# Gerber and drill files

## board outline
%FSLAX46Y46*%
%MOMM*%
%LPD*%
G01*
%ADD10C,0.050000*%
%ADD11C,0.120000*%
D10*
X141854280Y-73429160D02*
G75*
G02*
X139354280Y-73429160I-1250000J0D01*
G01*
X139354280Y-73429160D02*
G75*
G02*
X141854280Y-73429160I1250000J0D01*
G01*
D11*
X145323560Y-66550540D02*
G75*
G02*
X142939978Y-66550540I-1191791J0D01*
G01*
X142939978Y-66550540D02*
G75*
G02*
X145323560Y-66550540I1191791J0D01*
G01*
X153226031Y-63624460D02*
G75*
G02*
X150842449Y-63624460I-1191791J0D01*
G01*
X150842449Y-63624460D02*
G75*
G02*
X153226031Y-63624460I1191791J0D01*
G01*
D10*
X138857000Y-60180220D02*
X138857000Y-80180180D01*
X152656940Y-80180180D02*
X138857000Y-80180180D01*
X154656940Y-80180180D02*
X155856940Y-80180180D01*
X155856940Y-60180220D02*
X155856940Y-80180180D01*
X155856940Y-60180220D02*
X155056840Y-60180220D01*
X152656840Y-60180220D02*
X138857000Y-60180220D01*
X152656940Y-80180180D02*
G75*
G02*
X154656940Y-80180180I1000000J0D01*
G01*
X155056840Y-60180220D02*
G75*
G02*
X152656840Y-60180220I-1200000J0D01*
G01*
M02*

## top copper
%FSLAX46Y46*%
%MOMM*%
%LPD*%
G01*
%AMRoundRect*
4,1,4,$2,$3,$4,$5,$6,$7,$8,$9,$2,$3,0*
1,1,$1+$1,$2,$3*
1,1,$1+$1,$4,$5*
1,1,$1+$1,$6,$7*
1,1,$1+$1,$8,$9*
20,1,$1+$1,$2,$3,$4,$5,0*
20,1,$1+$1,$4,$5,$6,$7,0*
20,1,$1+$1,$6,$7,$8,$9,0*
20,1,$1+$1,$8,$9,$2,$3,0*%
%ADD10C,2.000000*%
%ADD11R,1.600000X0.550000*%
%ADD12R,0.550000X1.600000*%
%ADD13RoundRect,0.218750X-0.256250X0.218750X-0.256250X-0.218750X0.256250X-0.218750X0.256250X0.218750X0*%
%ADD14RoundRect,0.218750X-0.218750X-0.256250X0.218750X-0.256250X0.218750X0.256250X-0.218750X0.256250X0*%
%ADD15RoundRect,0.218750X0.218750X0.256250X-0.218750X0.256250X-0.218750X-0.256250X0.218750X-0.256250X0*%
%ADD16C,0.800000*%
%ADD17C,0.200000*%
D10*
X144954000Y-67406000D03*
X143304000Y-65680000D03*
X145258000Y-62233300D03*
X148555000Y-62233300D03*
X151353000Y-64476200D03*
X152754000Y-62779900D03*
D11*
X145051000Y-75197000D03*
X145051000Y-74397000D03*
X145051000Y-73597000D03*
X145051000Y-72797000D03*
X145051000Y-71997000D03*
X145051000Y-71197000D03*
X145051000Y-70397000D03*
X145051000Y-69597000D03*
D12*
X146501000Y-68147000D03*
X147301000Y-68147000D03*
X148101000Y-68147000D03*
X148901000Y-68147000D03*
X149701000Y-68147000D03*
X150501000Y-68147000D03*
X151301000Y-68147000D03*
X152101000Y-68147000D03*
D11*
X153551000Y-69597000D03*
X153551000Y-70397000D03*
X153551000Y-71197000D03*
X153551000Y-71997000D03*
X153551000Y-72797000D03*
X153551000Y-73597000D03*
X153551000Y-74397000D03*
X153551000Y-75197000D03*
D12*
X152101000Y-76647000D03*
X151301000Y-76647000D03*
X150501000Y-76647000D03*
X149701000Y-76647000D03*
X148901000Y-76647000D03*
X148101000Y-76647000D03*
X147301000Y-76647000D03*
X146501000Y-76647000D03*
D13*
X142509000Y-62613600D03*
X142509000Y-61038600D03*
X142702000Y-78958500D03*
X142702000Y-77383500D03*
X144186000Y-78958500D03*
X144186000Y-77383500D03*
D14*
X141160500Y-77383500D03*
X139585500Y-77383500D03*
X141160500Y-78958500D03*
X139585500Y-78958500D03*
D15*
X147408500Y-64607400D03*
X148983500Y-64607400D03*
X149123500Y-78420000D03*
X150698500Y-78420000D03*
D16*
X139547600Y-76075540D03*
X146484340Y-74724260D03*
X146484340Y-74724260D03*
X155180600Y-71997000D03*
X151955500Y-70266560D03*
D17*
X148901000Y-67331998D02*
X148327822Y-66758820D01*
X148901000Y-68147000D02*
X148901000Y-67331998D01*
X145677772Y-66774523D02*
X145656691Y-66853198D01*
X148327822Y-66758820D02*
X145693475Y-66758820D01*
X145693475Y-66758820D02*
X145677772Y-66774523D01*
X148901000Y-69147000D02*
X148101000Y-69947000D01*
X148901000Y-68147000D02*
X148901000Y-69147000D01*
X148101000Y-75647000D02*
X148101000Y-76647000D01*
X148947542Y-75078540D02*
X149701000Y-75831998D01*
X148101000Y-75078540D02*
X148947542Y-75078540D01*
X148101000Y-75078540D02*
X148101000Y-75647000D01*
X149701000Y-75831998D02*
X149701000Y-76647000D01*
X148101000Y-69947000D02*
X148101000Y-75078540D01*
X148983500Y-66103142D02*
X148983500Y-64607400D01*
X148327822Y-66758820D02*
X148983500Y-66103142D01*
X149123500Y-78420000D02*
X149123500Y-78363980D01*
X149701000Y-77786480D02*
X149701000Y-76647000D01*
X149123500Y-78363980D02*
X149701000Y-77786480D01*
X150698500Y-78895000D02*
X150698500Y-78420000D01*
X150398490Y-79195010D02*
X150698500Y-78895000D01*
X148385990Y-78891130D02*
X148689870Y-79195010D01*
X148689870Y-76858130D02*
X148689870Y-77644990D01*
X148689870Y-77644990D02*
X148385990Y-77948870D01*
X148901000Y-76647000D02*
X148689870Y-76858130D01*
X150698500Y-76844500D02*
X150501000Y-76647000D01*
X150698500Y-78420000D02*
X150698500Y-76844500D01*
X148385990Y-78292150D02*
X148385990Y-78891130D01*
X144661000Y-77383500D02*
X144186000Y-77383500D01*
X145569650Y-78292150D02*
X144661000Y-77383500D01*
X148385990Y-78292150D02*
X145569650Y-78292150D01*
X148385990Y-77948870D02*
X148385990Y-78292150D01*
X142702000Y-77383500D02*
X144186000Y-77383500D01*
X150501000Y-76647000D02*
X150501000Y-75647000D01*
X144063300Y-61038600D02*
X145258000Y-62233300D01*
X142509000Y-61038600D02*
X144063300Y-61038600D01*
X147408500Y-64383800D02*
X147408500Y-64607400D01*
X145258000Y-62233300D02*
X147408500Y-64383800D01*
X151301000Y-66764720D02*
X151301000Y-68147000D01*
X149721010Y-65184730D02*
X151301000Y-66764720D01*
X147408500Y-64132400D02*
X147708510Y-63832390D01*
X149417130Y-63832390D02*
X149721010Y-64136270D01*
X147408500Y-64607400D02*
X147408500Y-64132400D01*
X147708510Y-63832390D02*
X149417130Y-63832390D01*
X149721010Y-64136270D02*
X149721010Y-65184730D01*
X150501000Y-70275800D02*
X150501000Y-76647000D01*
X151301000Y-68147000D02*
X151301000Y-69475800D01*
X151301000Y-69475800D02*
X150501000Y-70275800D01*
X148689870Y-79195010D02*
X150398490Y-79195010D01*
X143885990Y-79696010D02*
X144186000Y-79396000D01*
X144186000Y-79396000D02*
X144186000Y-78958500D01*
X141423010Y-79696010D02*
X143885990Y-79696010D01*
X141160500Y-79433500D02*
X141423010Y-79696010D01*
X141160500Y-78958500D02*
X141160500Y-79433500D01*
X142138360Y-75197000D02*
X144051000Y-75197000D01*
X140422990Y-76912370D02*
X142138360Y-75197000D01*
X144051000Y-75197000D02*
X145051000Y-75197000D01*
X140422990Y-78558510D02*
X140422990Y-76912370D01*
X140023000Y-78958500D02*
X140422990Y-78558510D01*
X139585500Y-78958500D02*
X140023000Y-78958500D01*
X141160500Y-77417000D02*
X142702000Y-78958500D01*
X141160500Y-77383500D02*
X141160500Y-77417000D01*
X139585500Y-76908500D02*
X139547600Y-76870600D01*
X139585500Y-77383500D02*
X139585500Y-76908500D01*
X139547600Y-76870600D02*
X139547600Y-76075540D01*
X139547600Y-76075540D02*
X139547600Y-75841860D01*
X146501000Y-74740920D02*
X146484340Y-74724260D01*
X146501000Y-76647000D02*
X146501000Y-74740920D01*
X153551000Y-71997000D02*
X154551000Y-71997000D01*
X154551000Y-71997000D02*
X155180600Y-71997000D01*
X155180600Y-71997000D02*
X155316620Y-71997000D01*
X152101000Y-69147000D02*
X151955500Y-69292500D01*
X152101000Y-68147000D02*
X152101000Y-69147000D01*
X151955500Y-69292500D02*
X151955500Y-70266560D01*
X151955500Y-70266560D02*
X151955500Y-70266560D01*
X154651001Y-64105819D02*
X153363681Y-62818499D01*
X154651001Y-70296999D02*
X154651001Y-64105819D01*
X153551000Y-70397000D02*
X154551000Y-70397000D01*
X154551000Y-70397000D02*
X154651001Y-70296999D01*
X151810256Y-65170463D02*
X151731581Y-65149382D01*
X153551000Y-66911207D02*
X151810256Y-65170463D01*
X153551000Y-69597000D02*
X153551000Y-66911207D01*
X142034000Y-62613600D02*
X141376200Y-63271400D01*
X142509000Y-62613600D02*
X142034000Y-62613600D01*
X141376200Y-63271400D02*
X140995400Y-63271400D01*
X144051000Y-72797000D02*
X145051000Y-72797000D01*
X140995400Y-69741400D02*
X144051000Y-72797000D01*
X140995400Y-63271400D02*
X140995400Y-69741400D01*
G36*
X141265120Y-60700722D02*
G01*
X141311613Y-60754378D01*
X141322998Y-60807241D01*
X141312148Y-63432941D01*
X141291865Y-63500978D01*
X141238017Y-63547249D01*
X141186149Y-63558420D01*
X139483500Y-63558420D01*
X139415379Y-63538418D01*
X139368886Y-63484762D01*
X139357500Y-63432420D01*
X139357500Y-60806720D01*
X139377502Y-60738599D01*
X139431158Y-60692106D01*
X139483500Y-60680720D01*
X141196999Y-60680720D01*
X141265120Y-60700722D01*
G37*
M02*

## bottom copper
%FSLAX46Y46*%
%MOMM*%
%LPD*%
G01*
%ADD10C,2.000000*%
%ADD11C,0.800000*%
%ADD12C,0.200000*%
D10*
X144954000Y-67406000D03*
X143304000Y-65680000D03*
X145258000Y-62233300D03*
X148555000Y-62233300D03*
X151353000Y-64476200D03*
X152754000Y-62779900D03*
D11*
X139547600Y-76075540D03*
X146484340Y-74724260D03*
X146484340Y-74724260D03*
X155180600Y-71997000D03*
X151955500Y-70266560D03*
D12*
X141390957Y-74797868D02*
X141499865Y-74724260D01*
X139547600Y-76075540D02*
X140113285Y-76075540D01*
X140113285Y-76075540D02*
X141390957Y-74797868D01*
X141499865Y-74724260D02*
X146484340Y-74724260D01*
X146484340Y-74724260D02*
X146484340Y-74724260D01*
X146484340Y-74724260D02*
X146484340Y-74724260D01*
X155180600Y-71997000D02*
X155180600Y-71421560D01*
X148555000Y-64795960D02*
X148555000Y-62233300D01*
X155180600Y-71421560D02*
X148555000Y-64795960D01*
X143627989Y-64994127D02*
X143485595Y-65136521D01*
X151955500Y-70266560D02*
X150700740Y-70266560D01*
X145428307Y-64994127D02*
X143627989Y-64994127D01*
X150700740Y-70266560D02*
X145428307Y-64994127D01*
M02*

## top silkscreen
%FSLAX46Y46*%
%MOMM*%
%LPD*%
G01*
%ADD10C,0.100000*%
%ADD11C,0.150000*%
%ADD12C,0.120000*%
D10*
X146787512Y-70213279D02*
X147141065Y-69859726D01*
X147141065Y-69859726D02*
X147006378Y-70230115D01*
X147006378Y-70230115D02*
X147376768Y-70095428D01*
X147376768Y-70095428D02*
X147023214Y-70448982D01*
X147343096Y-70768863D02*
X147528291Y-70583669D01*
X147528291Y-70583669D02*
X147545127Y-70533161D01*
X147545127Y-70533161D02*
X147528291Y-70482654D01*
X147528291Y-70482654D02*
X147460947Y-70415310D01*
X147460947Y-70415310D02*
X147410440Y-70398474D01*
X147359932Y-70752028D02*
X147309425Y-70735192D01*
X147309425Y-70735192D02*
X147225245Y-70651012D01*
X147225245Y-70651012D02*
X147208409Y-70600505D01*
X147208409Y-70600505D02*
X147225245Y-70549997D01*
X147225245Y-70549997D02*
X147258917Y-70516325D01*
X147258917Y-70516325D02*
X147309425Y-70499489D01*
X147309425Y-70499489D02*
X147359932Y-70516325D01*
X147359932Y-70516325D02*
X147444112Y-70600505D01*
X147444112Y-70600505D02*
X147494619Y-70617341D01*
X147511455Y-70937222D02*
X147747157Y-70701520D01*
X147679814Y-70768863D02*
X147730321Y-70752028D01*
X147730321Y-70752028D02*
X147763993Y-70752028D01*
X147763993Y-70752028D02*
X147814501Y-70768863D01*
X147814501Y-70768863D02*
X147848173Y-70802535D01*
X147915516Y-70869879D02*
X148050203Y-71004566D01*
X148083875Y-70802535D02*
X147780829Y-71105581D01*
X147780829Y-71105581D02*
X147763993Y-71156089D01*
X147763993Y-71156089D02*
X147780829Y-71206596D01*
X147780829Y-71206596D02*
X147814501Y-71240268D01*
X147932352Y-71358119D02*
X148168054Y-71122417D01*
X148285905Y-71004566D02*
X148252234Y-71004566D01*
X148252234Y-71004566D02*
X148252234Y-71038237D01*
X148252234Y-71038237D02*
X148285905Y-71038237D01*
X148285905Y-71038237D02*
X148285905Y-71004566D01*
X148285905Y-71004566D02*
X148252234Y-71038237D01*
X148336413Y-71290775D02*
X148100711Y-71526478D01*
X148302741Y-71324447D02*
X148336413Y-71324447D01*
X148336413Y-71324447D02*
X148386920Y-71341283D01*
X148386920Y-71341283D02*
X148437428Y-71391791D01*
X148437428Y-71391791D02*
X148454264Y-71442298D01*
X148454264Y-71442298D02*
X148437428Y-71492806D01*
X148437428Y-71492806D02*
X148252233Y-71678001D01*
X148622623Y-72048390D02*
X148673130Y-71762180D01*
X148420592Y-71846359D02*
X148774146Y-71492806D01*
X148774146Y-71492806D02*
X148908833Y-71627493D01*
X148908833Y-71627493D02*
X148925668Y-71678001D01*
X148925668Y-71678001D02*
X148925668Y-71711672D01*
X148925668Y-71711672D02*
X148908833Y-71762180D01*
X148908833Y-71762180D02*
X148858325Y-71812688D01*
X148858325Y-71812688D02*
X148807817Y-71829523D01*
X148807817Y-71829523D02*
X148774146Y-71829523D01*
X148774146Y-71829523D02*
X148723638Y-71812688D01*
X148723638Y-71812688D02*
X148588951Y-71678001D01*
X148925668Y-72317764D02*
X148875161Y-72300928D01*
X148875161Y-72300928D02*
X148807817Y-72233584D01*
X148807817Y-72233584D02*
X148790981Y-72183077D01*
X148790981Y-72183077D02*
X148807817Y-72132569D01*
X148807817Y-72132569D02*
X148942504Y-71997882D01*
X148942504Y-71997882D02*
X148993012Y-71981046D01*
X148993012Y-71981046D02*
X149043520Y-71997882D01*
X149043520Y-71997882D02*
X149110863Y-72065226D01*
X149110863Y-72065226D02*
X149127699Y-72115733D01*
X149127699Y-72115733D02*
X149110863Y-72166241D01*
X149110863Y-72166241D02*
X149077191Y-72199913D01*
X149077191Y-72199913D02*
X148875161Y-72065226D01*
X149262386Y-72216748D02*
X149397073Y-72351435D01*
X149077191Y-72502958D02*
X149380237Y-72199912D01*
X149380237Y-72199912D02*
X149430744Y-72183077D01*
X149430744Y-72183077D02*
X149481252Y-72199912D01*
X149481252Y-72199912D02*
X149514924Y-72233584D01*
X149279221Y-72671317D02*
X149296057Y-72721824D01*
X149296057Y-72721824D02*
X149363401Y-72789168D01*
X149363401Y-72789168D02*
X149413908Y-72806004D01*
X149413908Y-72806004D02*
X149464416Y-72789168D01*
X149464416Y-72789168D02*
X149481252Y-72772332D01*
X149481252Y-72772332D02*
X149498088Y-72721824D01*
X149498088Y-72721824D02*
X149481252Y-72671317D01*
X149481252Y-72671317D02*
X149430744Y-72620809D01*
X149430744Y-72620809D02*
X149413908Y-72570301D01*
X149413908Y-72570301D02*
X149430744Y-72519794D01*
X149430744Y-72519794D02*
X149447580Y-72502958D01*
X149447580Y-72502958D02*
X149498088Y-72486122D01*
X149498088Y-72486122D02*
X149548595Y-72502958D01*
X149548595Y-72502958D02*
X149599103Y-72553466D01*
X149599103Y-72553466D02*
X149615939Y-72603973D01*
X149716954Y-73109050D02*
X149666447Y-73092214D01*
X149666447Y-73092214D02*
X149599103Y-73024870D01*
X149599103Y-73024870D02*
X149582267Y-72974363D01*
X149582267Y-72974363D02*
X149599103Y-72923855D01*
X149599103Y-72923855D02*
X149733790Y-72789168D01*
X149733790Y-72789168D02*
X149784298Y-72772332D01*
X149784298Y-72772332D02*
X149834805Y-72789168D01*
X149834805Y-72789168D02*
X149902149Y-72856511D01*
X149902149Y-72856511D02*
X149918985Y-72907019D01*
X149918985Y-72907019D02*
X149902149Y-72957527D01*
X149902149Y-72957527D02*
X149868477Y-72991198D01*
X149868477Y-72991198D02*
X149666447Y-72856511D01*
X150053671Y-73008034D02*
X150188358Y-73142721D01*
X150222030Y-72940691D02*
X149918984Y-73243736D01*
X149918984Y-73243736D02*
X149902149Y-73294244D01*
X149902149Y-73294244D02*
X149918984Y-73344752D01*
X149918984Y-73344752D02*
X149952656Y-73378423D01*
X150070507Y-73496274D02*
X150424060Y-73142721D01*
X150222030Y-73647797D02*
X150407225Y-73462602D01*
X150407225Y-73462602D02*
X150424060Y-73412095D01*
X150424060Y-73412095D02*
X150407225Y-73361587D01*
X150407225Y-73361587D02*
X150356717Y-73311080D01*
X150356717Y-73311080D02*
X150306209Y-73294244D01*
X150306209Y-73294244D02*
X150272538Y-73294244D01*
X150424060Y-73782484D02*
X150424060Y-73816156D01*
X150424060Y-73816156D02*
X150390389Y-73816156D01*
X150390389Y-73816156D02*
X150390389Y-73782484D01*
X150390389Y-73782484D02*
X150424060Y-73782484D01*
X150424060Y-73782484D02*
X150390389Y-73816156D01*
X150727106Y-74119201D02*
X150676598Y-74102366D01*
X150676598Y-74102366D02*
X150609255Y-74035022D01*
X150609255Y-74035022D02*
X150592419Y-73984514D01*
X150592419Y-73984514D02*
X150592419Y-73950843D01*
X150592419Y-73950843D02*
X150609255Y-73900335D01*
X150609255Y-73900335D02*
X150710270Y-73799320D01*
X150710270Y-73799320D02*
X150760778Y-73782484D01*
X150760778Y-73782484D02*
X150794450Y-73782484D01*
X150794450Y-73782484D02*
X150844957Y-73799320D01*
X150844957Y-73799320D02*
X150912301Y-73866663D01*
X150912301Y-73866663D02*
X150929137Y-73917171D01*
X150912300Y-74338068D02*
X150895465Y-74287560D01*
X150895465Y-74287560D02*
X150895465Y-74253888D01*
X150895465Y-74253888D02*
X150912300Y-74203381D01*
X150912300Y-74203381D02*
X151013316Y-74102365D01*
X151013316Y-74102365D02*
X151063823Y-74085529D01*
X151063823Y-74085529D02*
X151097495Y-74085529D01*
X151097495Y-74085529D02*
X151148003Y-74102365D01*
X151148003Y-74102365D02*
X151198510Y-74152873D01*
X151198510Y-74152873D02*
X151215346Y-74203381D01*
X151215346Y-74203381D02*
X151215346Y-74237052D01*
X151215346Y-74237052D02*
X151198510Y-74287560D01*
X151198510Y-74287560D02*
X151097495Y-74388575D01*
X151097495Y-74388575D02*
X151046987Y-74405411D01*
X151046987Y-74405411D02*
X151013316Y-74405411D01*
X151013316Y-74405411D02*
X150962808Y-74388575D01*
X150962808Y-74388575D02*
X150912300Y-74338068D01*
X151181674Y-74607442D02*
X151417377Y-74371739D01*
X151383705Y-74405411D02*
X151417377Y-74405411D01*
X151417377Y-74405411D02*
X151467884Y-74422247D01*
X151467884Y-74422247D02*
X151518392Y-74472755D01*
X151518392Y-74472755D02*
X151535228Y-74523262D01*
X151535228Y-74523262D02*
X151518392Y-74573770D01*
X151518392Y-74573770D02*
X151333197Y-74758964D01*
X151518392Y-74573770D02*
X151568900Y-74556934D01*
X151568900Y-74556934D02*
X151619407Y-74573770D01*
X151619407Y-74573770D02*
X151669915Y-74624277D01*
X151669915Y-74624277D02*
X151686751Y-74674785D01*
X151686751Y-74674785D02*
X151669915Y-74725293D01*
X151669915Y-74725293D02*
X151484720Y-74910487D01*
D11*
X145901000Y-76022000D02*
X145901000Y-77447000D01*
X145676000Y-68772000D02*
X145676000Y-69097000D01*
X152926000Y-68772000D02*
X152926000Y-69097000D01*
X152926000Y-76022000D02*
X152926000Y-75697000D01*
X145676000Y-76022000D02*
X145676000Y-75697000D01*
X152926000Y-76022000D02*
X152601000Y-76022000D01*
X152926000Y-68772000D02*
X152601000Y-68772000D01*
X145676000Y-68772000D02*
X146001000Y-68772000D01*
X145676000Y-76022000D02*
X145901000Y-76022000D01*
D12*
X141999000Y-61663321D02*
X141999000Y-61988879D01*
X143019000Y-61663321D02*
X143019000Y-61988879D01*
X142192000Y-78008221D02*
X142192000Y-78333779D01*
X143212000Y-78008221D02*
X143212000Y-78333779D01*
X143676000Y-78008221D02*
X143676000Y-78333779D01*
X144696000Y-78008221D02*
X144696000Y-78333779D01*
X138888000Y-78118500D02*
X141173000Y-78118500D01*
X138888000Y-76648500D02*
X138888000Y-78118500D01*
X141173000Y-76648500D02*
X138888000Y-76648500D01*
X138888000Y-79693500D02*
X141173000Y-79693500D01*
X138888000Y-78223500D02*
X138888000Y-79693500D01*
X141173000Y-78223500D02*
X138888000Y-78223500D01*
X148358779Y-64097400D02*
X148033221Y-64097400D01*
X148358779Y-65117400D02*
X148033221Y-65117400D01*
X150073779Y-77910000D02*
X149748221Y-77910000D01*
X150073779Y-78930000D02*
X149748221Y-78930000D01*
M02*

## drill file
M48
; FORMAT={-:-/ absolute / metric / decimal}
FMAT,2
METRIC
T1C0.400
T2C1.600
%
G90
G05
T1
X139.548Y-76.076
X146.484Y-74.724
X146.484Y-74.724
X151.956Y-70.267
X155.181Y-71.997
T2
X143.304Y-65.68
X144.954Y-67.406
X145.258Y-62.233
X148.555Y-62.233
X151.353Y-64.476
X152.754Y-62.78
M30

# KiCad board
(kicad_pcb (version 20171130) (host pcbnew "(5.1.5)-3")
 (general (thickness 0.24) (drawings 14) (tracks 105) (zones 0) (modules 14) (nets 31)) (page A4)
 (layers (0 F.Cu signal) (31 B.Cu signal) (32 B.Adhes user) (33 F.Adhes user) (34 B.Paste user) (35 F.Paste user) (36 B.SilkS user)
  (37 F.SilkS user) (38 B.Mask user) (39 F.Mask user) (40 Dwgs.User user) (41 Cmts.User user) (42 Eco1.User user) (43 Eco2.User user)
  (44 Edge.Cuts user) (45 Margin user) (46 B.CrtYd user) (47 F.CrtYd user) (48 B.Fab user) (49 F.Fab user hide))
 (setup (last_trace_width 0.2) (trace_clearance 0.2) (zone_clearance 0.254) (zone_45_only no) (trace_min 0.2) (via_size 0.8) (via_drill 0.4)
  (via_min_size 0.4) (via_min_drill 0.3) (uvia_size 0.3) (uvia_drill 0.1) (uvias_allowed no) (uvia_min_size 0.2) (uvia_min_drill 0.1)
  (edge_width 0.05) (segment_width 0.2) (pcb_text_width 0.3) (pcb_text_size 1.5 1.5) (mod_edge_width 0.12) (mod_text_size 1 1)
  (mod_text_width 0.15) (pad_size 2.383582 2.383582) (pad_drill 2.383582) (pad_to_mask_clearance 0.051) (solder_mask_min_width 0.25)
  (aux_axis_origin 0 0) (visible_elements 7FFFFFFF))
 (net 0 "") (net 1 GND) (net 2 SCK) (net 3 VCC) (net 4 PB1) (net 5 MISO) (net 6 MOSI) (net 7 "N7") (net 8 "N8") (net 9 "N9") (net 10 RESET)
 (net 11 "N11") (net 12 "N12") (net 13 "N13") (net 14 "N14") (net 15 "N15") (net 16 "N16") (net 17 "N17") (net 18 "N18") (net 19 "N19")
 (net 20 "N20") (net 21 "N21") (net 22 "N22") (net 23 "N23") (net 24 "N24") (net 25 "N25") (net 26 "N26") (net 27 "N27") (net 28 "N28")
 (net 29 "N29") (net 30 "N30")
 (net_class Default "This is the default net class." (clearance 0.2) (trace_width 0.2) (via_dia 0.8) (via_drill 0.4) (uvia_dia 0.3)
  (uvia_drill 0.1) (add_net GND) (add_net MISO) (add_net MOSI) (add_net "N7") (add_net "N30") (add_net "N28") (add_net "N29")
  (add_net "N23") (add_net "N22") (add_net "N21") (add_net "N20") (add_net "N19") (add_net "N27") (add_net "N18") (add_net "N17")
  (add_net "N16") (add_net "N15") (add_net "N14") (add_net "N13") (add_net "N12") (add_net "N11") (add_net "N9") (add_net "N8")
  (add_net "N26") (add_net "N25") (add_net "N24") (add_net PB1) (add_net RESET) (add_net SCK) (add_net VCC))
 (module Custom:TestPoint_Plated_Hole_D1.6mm (layer F.Cu) (at 144.954 67.406 180)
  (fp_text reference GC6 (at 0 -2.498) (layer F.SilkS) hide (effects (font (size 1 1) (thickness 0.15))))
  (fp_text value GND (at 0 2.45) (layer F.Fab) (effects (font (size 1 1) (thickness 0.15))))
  (pad 1 thru_hole circle (at 0 0 180) (size 2 2) (drill 1.6) (layers *.Cu *.Mask) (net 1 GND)))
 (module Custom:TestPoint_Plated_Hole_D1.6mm (layer F.Cu) (at 143.304 65.68 180)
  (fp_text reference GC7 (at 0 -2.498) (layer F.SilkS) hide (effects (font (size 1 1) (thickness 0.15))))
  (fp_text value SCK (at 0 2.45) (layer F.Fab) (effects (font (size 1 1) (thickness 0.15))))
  (pad 1 thru_hole circle (at 0 0 180) (size 2 2) (drill 1.6) (layers *.Cu *.Mask) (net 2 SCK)))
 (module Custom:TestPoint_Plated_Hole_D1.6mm (layer F.Cu) (at 145.258 62.2333 180)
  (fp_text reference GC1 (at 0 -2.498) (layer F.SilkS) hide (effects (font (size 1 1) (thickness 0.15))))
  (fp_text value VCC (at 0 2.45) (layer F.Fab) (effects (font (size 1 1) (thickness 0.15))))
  (pad 1 thru_hole circle (at 0 0 180) (size 2 2) (drill 1.6) (layers *.Cu *.Mask) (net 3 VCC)))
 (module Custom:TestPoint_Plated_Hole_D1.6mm (layer F.Cu) (at 148.555 62.2333 180)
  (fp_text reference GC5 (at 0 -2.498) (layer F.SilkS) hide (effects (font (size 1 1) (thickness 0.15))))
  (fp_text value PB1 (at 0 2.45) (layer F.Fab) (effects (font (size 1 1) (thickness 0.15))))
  (pad 1 thru_hole circle (at 0 0 180) (size 2 2) (drill 1.6) (layers *.Cu *.Mask) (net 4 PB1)))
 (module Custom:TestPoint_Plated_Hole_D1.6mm (layer F.Cu) (at 151.353 64.4762 180)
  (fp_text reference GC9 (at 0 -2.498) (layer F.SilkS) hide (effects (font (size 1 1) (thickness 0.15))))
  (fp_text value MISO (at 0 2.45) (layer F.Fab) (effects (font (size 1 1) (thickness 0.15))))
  (pad 1 thru_hole circle (at 0 0 180) (size 2 2) (drill 1.6) (layers *.Cu *.Mask) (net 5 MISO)))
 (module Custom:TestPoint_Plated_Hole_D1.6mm (layer F.Cu) (at 152.754 62.7799 180)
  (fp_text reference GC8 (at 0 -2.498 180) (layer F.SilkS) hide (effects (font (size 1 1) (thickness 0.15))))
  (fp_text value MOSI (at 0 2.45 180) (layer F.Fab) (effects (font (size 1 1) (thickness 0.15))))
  (pad 1 thru_hole circle (at 0 0 180) (size 2 2) (drill 1.6) (layers *.Cu *.Mask) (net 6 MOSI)))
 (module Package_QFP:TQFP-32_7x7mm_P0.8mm (layer F.Cu) (at 149.301 72.397 90)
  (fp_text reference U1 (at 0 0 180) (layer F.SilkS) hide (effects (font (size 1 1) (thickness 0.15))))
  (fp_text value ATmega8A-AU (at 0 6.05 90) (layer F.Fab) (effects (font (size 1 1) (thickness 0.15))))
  (fp_line (start -3.625 -3.4) (end -5.05 -3.4) (layer F.SilkS) (width 0.15))
  (fp_line (start 3.625 -3.625) (end 3.3 -3.625) (layer F.SilkS) (width 0.15))
  (fp_line (start 3.625 3.625) (end 3.3 3.625) (layer F.SilkS) (width 0.15))
  (fp_line (start -3.625 3.625) (end -3.3 3.625) (layer F.SilkS) (width 0.15))
  (fp_line (start -3.625 -3.625) (end -3.3 -3.625) (layer F.SilkS) (width 0.15))
  (fp_line (start -3.625 3.625) (end -3.625 3.3) (layer F.SilkS) (width 0.15))
  (fp_line (start 3.625 3.625) (end 3.625 3.3) (layer F.SilkS) (width 0.15))
  (fp_line (start 3.625 -3.625) (end 3.625 -3.3) (layer F.SilkS) (width 0.15))
  (fp_line (start -3.625 -3.625) (end -3.625 -3.4) (layer F.SilkS) (width 0.15))
  (pad 32 smd rect (at -2.8 -4.25 180) (size 1.6 0.55) (layers F.Cu F.Paste F.Mask) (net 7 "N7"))
  (pad 31 smd rect (at -2 -4.25 180) (size 1.6 0.55) (layers F.Cu F.Paste F.Mask) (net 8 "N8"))
  (pad 30 smd rect (at -1.2 -4.25 180) (size 1.6 0.55) (layers F.Cu F.Paste F.Mask) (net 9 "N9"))
  (pad 29 smd rect (at -0.4 -4.25 180) (size 1.6 0.55) (layers F.Cu F.Paste F.Mask) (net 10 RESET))
  (pad 28 smd rect (at 0.4 -4.25 180) (size 1.6 0.55) (layers F.Cu F.Paste F.Mask) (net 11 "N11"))
  (pad 27 smd rect (at 1.2 -4.25 180) (size 1.6 0.55) (layers F.Cu F.Paste F.Mask) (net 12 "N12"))
  (pad 26 smd rect (at 2 -4.25 180) (size 1.6 0.55) (layers F.Cu F.Paste F.Mask) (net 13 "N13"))
  (pad 25 smd rect (at 2.8 -4.25 180) (size 1.6 0.55) (layers F.Cu F.Paste F.Mask) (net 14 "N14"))
  (pad 24 smd rect (at 4.25 -2.8 90) (size 1.6 0.55) (layers F.Cu F.Paste F.Mask) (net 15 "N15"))
  (pad 23 smd rect (at 4.25 -2 90) (size 1.6 0.55) (layers F.Cu F.Paste F.Mask) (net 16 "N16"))
  (pad 22 smd rect (at 4.25 -1.2 90) (size 1.6 0.55) (layers F.Cu F.Paste F.Mask) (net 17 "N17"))
  (pad 21 smd rect (at 4.25 -0.4 90) (size 1.6 0.55) (layers F.Cu F.Paste F.Mask) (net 1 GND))
  (pad 20 smd rect (at 4.25 0.4 90) (size 1.6 0.55) (layers F.Cu F.Paste F.Mask) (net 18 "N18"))
  (pad 19 smd rect (at 4.25 1.2 90) (size 1.6 0.55) (layers F.Cu F.Paste F.Mask) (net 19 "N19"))
  (pad 18 smd rect (at 4.25 2 90) (size 1.6 0.55) (layers F.Cu F.Paste F.Mask) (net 3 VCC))
  (pad 17 smd rect (at 4.25 2.8 90) (size 1.6 0.55) (layers F.Cu F.Paste F.Mask) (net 2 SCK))
  (pad 16 smd rect (at 2.8 4.25 180) (size 1.6 0.55) (layers F.Cu F.Paste F.Mask) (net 5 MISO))
  (pad 15 smd rect (at 2 4.25 180) (size 1.6 0.55) (layers F.Cu F.Paste F.Mask) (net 6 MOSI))
  (pad 14 smd rect (at 1.2 4.25 180) (size 1.6 0.55) (layers F.Cu F.Paste F.Mask) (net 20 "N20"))
  (pad 13 smd rect (at 0.4 4.25 180) (size 1.6 0.55) (layers F.Cu F.Paste F.Mask) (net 4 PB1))
  (pad 12 smd rect (at -0.4 4.25 180) (size 1.6 0.55) (layers F.Cu F.Paste F.Mask) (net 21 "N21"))
  (pad 11 smd rect (at -1.2 4.25 180) (size 1.6 0.55) (layers F.Cu F.Paste F.Mask) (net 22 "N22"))
  (pad 10 smd rect (at -2 4.25 180) (size 1.6 0.55) (layers F.Cu F.Paste F.Mask) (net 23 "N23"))
  (pad 9 smd rect (at -2.8 4.25 180) (size 1.6 0.55) (layers F.Cu F.Paste F.Mask) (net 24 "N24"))
  (pad 8 smd rect (at -4.25 2.8 90) (size 1.6 0.55) (layers F.Cu F.Paste F.Mask) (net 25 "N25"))
  (pad 7 smd rect (at -4.25 2 90) (size 1.6 0.55) (layers F.Cu F.Paste F.Mask) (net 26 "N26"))
  (pad 6 smd rect (at -4.25 1.2 90) (size 1.6 0.55) (layers F.Cu F.Paste F.Mask) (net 3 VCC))
  (pad 5 smd rect (at -4.25 0.4 90) (size 1.6 0.55) (layers F.Cu F.Paste F.Mask) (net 1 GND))
  (pad 4 smd rect (at -4.25 -0.4 90) (size 1.6 0.55) (layers F.Cu F.Paste F.Mask) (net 3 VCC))
  (pad 3 smd rect (at -4.25 -1.2 90) (size 1.6 0.55) (layers F.Cu F.Paste F.Mask) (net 1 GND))
  (pad 2 smd rect (at -4.25 -2 90) (size 1.6 0.55) (layers F.Cu F.Paste F.Mask) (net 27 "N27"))
  (pad 1 smd rect (at -4.25 -2.8 90) (size 1.6 0.55) (layers F.Cu F.Paste F.Mask) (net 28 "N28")))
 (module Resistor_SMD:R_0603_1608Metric (layer F.Cu) (at 142.509 61.8261 270)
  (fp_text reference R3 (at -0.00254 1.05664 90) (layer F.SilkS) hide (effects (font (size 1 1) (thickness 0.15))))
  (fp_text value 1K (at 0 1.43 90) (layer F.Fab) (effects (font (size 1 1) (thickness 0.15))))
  (fp_line (start -0.162779 0.51) (end 0.162779 0.51) (layer F.SilkS) (width 0.12))
  (fp_line (start -0.162779 -0.51) (end 0.162779 -0.51) (layer F.SilkS) (width 0.12))
  (pad 2 smd roundrect (at 0.7875 0 270) (size 0.875 0.95) (layers F.Cu F.Paste F.Mask) (roundrect_rratio 0.25) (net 10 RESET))
  (pad 1 smd roundrect (at -0.7875 0 270) (size 0.875 0.95) (layers F.Cu F.Paste F.Mask) (roundrect_rratio 0.25) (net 3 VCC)))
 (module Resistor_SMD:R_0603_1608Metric (layer F.Cu) (at 142.702 78.171 270)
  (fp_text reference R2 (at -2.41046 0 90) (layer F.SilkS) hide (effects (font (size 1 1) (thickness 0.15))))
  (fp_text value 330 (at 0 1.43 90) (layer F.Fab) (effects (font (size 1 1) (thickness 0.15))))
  (fp_line (start -0.162779 0.51) (end 0.162779 0.51) (layer F.SilkS) (width 0.12))
  (fp_line (start -0.162779 -0.51) (end 0.162779 -0.51) (layer F.SilkS) (width 0.12))
  (pad 2 smd roundrect (at 0.7875 0 270) (size 0.875 0.95) (layers F.Cu F.Paste F.Mask) (roundrect_rratio 0.25) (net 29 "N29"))
  (pad 1 smd roundrect (at -0.7875 0 270) (size 0.875 0.95) (layers F.Cu F.Paste F.Mask) (roundrect_rratio 0.25) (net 3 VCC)))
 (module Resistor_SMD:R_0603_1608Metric (layer F.Cu) (at 144.186 78.171 270)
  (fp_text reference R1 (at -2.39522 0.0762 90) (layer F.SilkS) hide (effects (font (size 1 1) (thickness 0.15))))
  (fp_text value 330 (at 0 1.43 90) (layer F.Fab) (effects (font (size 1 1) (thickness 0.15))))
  (fp_line (start -0.162779 0.51) (end 0.162779 0.51) (layer F.SilkS) (width 0.12))
  (fp_line (start -0.162779 -0.51) (end 0.162779 -0.51) (layer F.SilkS) (width 0.12))
  (pad 2 smd roundrect (at 0.7875 0 270) (size 0.875 0.95) (layers F.Cu F.Paste F.Mask) (roundrect_rratio 0.25) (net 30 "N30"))
  (pad 1 smd roundrect (at -0.7875 0 270) (size 0.875 0.95) (layers F.Cu F.Paste F.Mask) (roundrect_rratio 0.25) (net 3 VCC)))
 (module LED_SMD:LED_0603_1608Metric (layer F.Cu) (at 140.373 77.3835)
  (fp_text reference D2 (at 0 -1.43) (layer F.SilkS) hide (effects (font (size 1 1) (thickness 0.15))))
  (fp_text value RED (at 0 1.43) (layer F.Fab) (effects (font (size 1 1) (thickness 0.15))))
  (fp_line (start -1.485 0.735) (end 0.8 0.735) (layer F.SilkS) (width 0.12))
  (fp_line (start -1.485 -0.735) (end -1.485 0.735) (layer F.SilkS) (width 0.12))
  (fp_line (start 0.8 -0.735) (end -1.485 -0.735) (layer F.SilkS) (width 0.12))
  (pad 2 smd roundrect (at 0.7875 0) (size 0.875 0.95) (layers F.Cu F.Paste F.Mask) (roundrect_rratio 0.25) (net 29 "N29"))
  (pad 1 smd roundrect (at -0.7875 0) (size 0.875 0.95) (layers F.Cu F.Paste F.Mask) (roundrect_rratio 0.25) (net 28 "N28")))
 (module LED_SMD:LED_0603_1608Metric (layer F.Cu) (at 140.373 78.9585)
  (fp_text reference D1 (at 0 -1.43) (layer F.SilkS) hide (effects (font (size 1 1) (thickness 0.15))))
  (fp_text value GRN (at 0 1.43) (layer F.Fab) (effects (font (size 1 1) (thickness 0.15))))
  (fp_line (start -1.485 0.735) (end 0.8 0.735) (layer F.SilkS) (width 0.12))
  (fp_line (start -1.485 -0.735) (end -1.485 0.735) (layer F.SilkS) (width 0.12))
  (fp_line (start 0.8 -0.735) (end -1.485 -0.735) (layer F.SilkS) (width 0.12))
  (pad 2 smd roundrect (at 0.7875 0) (size 0.875 0.95) (layers F.Cu F.Paste F.Mask) (roundrect_rratio 0.25) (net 30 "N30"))
  (pad 1 smd roundrect (at -0.7875 0) (size 0.875 0.95) (layers F.Cu F.Paste F.Mask) (roundrect_rratio 0.25) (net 7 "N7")))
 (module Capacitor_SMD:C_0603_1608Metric (layer F.Cu) (at 148.196 64.6074 180)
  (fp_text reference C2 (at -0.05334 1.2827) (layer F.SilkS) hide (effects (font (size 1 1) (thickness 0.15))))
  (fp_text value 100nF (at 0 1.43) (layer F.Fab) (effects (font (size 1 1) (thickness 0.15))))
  (fp_line (start -0.162779 0.51) (end 0.162779 0.51) (layer F.SilkS) (width 0.12))
  (fp_line (start -0.162779 -0.51) (end 0.162779 -0.51) (layer F.SilkS) (width 0.12))
  (pad 2 smd roundrect (at 0.7875 0 180) (size 0.875 0.95) (layers F.Cu F.Paste F.Mask) (roundrect_rratio 0.25) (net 3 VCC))
  (pad 1 smd roundrect (at -0.7875 0 180) (size 0.875 0.95) (layers F.Cu F.Paste F.Mask) (roundrect_rratio 0.25) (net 1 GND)))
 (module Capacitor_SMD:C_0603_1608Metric (layer F.Cu) (at 149.911 78.42 180)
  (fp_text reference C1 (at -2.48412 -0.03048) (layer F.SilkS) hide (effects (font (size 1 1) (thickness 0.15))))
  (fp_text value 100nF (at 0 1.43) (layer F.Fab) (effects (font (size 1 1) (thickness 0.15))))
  (fp_line (start -0.162779 0.51) (end 0.162779 0.51) (layer F.SilkS) (width 0.12))
  (fp_line (start -0.162779 -0.51) (end 0.162779 -0.51) (layer F.SilkS) (width 0.12))
  (pad 2 smd roundrect (at 0.7875 0 180) (size 0.875 0.95) (layers F.Cu F.Paste F.Mask) (roundrect_rratio 0.25) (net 1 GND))
  (pad 1 smd roundrect (at -0.7875 0 180) (size 0.875 0.95) (layers F.Cu F.Paste F.Mask) (roundrect_rratio 0.25) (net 3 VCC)))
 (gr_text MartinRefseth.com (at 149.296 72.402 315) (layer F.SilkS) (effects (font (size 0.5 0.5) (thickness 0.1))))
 (gr_circle (center 140.60428 73.42916) (end 140.60428 74.67916) (layer Edge.Cuts) (width 0.05))
 (gr_circle (center 144.131769 66.55054) (end 144.131769 65.358749) (layer Edge.Cuts) (width 0.12))
 (gr_circle (center 152.03424 63.62446) (end 152.03424 62.432669) (layer Edge.Cuts) (width 0.12))
 (gr_line (start 138.857 60.18022) (end 138.857 80.18018) (layer Edge.Cuts) (width 0.05))
 (gr_line (start 152.65694 80.18018) (end 138.857 80.18018) (layer Edge.Cuts) (width 0.05))
 (gr_line (start 154.65694 80.18018) (end 155.85694 80.18018) (layer Edge.Cuts) (width 0.05))
 (gr_line (start 155.85694 60.18022) (end 155.85694 80.18018) (layer Edge.Cuts) (width 0.05))
 (gr_line (start 155.85694 60.18022) (end 155.05684 60.18022) (layer Edge.Cuts) (width 0.05))
 (gr_line (start 152.65684 60.18022) (end 138.857 60.18022) (layer Edge.Cuts) (width 0.05))
 (gr_arc (start 153.65694 80.18018) (end 154.65694 80.18018) (angle -180) (layer Edge.Cuts) (width 0.05))
 (gr_arc (start 153.85684 60.18022) (end 152.65684 60.18022) (angle -180) (layer Edge.Cuts) (width 0.05))
 (segment (start 148.901 67.331998) (end 148.327822 66.75882) (width 0.2) (layer F.Cu) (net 1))
 (segment (start 148.901 68.147) (end 148.901 67.331998) (width 0.2) (layer F.Cu) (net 1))
 (segment (start 145.677772 66.774523) (end 145.656691 66.853198) (width 0.2) (layer F.Cu) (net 1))
 (segment (start 148.327822 66.75882) (end 145.693475 66.75882) (width 0.2) (layer F.Cu) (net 1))
 (segment (start 145.693475 66.75882) (end 145.677772 66.774523) (width 0.2) (layer F.Cu) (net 1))
 (segment (start 148.901 69.147) (end 148.101 69.947) (width 0.2) (layer F.Cu) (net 1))
 (segment (start 148.901 68.147) (end 148.901 69.147) (width 0.2) (layer F.Cu) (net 1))
 (segment (start 148.101 75.647) (end 148.101 76.647) (width 0.2) (layer F.Cu) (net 1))
 (segment (start 148.947542 75.07854) (end 149.701 75.831998) (width 0.2) (layer F.Cu) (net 1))
 (segment (start 148.101 75.07854) (end 148.947542 75.07854) (width 0.2) (layer F.Cu) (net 1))
 (segment (start 148.101 75.07854) (end 148.101 75.647) (width 0.2) (layer F.Cu) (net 1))
 (segment (start 149.701 75.831998) (end 149.701 76.647) (width 0.2) (layer F.Cu) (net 1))
 (segment (start 148.101 69.947) (end 148.101 75.07854) (width 0.2) (layer F.Cu) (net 1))
 (segment (start 148.9835 66.103142) (end 148.9835 64.6074) (width 0.2) (layer F.Cu) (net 1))
 (segment (start 148.327822 66.75882) (end 148.9835 66.103142) (width 0.2) (layer F.Cu) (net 1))
 (segment (start 149.1235 78.42) (end 149.1235 78.36398) (width 0.2) (layer F.Cu) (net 1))
 (segment (start 149.701 77.78648) (end 149.701 76.647) (width 0.2) (layer F.Cu) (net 1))
 (segment (start 149.1235 78.36398) (end 149.701 77.78648) (width 0.2) (layer F.Cu) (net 1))
 (segment (start 150.6985 78.895) (end 150.6985 78.42) (width 0.2) (layer F.Cu) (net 3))
 (segment (start 150.39849 79.19501) (end 150.6985 78.895) (width 0.2) (layer F.Cu) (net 3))
 (segment (start 148.38599 78.89113) (end 148.68987 79.19501) (width 0.2) (layer F.Cu) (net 3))
 (segment (start 148.68987 76.85813) (end 148.68987 77.64499) (width 0.2) (layer F.Cu) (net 3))
 (segment (start 148.68987 77.64499) (end 148.38599 77.94887) (width 0.2) (layer F.Cu) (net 3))
 (segment (start 148.901 76.647) (end 148.68987 76.85813) (width 0.2) (layer F.Cu) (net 3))
 (segment (start 150.6985 76.8445) (end 150.501 76.647) (width 0.2) (layer F.Cu) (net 3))
 (segment (start 150.6985 78.42) (end 150.6985 76.8445) (width 0.2) (layer F.Cu) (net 3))
 (segment (start 148.38599 78.29215) (end 148.38599 78.89113) (width 0.2) (layer F.Cu) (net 3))
 (segment (start 144.661 77.3835) (end 144.186 77.3835) (width 0.2) (layer F.Cu) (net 3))
 (segment (start 145.56965 78.29215) (end 144.661 77.3835) (width 0.2) (layer F.Cu) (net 3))
 (segment (start 148.38599 78.29215) (end 145.56965 78.29215) (width 0.2) (layer F.Cu) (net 3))
 (segment (start 148.38599 77.94887) (end 148.38599 78.29215) (width 0.2) (layer F.Cu) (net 3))
 (segment (start 142.702 77.3835) (end 144.186 77.3835) (width 0.2) (layer F.Cu) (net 3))
 (segment (start 150.501 76.647) (end 150.501 75.647) (width 0.2) (layer F.Cu) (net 3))
 (segment (start 144.0633 61.0386) (end 145.258 62.2333) (width 0.2) (layer F.Cu) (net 3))
 (segment (start 142.509 61.0386) (end 144.0633 61.0386) (width 0.2) (layer F.Cu) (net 3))
 (segment (start 147.4085 64.3838) (end 147.4085 64.6074) (width 0.2) (layer F.Cu) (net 3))
 (segment (start 145.258 62.2333) (end 147.4085 64.3838) (width 0.2) (layer F.Cu) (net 3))
 (segment (start 151.301 66.76472) (end 151.301 68.147) (width 0.2) (layer F.Cu) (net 3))
 (segment (start 149.72101 65.18473) (end 151.301 66.76472) (width 0.2) (layer F.Cu) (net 3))
 (segment (start 147.4085 64.1324) (end 147.70851 63.83239) (width 0.2) (layer F.Cu) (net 3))
 (segment (start 149.41713 63.83239) (end 149.72101 64.13627) (width 0.2) (layer F.Cu) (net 3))
 (segment (start 147.4085 64.6074) (end 147.4085 64.1324) (width 0.2) (layer F.Cu) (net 3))
 (segment (start 147.70851 63.83239) (end 149.41713 63.83239) (width 0.2) (layer F.Cu) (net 3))
 (segment (start 149.72101 64.13627) (end 149.72101 65.18473) (width 0.2) (layer F.Cu) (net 3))
 (segment (start 150.501 70.2758) (end 150.501 76.647) (width 0.2) (layer F.Cu) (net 3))
 (segment (start 151.301 68.147) (end 151.301 69.4758) (width 0.2) (layer F.Cu) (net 3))
 (segment (start 151.301 69.4758) (end 150.501 70.2758) (width 0.2) (layer F.Cu) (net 3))
 (segment (start 148.68987 79.19501) (end 150.39849 79.19501) (width 0.2) (layer F.Cu) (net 3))
 (segment (start 143.88599 79.69601) (end 144.186 79.396) (width 0.2) (layer F.Cu) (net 30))
 (segment (start 144.186 79.396) (end 144.186 78.9585) (width 0.2) (layer F.Cu) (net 30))
 (segment (start 141.42301 79.69601) (end 143.88599 79.69601) (width 0.2) (layer F.Cu) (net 30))
 (segment (start 141.1605 79.4335) (end 141.42301 79.69601) (width 0.2) (layer F.Cu) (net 30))
 (segment (start 141.1605 78.9585) (end 141.1605 79.4335) (width 0.2) (layer F.Cu) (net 30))
 (segment (start 142.13836 75.197) (end 144.051 75.197) (width 0.2) (layer F.Cu) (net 7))
 (segment (start 140.42299 76.91237) (end 142.13836 75.197) (width 0.2) (layer F.Cu) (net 7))
 (segment (start 144.051 75.197) (end 145.051 75.197) (width 0.2) (layer F.Cu) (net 7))
 (segment (start 140.42299 78.55851) (end 140.42299 76.91237) (width 0.2) (layer F.Cu) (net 7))
 (segment (start 140.023 78.9585) (end 140.42299 78.55851) (width 0.2) (layer F.Cu) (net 7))
 (segment (start 139.5855 78.9585) (end 140.023 78.9585) (width 0.2) (layer F.Cu) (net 7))
 (segment (start 141.1605 77.417) (end 142.702 78.9585) (width 0.2) (layer F.Cu) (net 29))
 (segment (start 141.1605 77.3835) (end 141.1605 77.417) (width 0.2) (layer F.Cu) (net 29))
 (segment (start 139.5855 76.9085) (end 139.5476 76.8706) (width 0.2) (layer F.Cu) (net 28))
 (segment (start 139.5855 77.3835) (end 139.5855 76.9085) (width 0.2) (layer F.Cu) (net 28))
 (segment (start 139.5476 76.8706) (end 139.5476 76.07554) (width 0.2) (layer F.Cu) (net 28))
 (segment (start 139.5476 76.07554) (end 139.5476 75.84186) (width 0.2) (layer F.Cu) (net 28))
 (via (at 139.5476 76.07554) (size 0.8) (drill 0.4) (layers F.Cu B.Cu) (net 28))
 (segment (start 141.390957 74.797868) (end 141.499865 74.72426) (width 0.2) (layer B.Cu) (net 28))
 (segment (start 139.5476 76.07554) (end 140.113285 76.07554) (width 0.2) (layer B.Cu) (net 28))
 (segment (start 140.113285 76.07554) (end 141.390957 74.797868) (width 0.2) (layer B.Cu) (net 28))
 (segment (start 141.499865 74.72426) (end 146.48434 74.72426) (width 0.2) (layer B.Cu) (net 28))
 (segment (start 146.48434 74.72426) (end 146.48434 74.72426) (width 0.2) (layer B.Cu) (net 28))
 (via (at 146.48434 74.72426) (size 0.8) (drill 0.4) (layers F.Cu B.Cu) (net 28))
 (segment (start 146.48434 74.72426) (end 146.48434 74.72426) (width 0.2) (layer B.Cu) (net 28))
 (via (at 146.48434 74.72426) (size 0.8) (drill 0.4) (layers F.Cu B.Cu) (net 28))
 (segment (start 146.501 74.74092) (end 146.48434 74.72426) (width 0.2) (layer F.Cu) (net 28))
 (segment (start 146.501 76.647) (end 146.501 74.74092) (width 0.2) (layer F.Cu) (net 28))
 (segment (start 153.551 71.997) (end 154.551 71.997) (width 0.2) (layer F.Cu) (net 4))
 (segment (start 154.551 71.997) (end 155.1806 71.997) (width 0.2) (layer F.Cu) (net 4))
 (segment (start 155.1806 71.997) (end 155.31662 71.997) (width 0.2) (layer F.Cu) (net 4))
 (via (at 155.1806 71.997) (size 0.8) (drill 0.4) (layers F.Cu B.Cu) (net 4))
 (segment (start 155.1806 71.997) (end 155.1806 71.42156) (width 0.2) (layer B.Cu) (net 4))
 (segment (start 148.555 64.79596) (end 148.555 62.2333) (width 0.2) (layer B.Cu) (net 4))
 (segment (start 155.1806 71.42156) (end 148.555 64.79596) (width 0.2) (layer B.Cu) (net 4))
 (segment (start 143.627989 64.994127) (end 143.485595 65.136521) (width 0.2) (layer B.Cu) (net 2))
 (segment (start 152.101 69.147) (end 151.9555 69.2925) (width 0.2) (layer F.Cu) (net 2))
 (segment (start 152.101 68.147) (end 152.101 69.147) (width 0.2) (layer F.Cu) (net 2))
 (segment (start 151.9555 69.2925) (end 151.9555 70.26656) (width 0.2) (layer F.Cu) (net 2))
 (segment (start 151.9555 70.26656) (end 151.9555 70.26656) (width 0.2) (layer F.Cu) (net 2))
 (via (at 151.9555 70.26656) (size 0.8) (drill 0.4) (layers F.Cu B.Cu) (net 2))
 (segment (start 151.9555 70.26656) (end 150.70074 70.26656) (width 0.2) (layer B.Cu) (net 2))
 (segment (start 145.428307 64.994127) (end 143.627989 64.994127) (width 0.2) (layer B.Cu) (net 2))
 (segment (start 150.70074 70.26656) (end 145.428307 64.994127) (width 0.2) (layer B.Cu) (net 2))
 (segment (start 154.651001 64.105819) (end 153.363681 62.818499) (width 0.2) (layer F.Cu) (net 6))
 (segment (start 154.651001 70.296999) (end 154.651001 64.105819) (width 0.2) (layer F.Cu) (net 6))
 (segment (start 153.551 70.397) (end 154.551 70.397) (width 0.2) (layer F.Cu) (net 6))
 (segment (start 154.551 70.397) (end 154.651001 70.296999) (width 0.2) (layer F.Cu) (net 6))
 (segment (start 151.810256 65.170463) (end 151.731581 65.149382) (width 0.2) (layer F.Cu) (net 5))
 (segment (start 153.551 66.911207) (end 151.810256 65.170463) (width 0.2) (layer F.Cu) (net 5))
 (segment (start 153.551 69.597) (end 153.551 66.911207) (width 0.2) (layer F.Cu) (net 5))
 (segment (start 142.034 62.6136) (end 141.3762 63.2714) (width 0.2) (layer F.Cu) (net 10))
 (segment (start 142.509 62.6136) (end 142.034 62.6136) (width 0.2) (layer F.Cu) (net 10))
 (segment (start 141.3762 63.2714) (end 140.9954 63.2714) (width 0.2) (layer F.Cu) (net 10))
 (segment (start 144.051 72.797) (end 145.051 72.797) (width 0.2) (layer F.Cu) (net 10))
 (segment (start 140.9954 69.7414) (end 144.051 72.797) (width 0.2) (layer F.Cu) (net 10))
 (segment (start 140.9954 63.2714) (end 140.9954 69.7414) (width 0.2) (layer F.Cu) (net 10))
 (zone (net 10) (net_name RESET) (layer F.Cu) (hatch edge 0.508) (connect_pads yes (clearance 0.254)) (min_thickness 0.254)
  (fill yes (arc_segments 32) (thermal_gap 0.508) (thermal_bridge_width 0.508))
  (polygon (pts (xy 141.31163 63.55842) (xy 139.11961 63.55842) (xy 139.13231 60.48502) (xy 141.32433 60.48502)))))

